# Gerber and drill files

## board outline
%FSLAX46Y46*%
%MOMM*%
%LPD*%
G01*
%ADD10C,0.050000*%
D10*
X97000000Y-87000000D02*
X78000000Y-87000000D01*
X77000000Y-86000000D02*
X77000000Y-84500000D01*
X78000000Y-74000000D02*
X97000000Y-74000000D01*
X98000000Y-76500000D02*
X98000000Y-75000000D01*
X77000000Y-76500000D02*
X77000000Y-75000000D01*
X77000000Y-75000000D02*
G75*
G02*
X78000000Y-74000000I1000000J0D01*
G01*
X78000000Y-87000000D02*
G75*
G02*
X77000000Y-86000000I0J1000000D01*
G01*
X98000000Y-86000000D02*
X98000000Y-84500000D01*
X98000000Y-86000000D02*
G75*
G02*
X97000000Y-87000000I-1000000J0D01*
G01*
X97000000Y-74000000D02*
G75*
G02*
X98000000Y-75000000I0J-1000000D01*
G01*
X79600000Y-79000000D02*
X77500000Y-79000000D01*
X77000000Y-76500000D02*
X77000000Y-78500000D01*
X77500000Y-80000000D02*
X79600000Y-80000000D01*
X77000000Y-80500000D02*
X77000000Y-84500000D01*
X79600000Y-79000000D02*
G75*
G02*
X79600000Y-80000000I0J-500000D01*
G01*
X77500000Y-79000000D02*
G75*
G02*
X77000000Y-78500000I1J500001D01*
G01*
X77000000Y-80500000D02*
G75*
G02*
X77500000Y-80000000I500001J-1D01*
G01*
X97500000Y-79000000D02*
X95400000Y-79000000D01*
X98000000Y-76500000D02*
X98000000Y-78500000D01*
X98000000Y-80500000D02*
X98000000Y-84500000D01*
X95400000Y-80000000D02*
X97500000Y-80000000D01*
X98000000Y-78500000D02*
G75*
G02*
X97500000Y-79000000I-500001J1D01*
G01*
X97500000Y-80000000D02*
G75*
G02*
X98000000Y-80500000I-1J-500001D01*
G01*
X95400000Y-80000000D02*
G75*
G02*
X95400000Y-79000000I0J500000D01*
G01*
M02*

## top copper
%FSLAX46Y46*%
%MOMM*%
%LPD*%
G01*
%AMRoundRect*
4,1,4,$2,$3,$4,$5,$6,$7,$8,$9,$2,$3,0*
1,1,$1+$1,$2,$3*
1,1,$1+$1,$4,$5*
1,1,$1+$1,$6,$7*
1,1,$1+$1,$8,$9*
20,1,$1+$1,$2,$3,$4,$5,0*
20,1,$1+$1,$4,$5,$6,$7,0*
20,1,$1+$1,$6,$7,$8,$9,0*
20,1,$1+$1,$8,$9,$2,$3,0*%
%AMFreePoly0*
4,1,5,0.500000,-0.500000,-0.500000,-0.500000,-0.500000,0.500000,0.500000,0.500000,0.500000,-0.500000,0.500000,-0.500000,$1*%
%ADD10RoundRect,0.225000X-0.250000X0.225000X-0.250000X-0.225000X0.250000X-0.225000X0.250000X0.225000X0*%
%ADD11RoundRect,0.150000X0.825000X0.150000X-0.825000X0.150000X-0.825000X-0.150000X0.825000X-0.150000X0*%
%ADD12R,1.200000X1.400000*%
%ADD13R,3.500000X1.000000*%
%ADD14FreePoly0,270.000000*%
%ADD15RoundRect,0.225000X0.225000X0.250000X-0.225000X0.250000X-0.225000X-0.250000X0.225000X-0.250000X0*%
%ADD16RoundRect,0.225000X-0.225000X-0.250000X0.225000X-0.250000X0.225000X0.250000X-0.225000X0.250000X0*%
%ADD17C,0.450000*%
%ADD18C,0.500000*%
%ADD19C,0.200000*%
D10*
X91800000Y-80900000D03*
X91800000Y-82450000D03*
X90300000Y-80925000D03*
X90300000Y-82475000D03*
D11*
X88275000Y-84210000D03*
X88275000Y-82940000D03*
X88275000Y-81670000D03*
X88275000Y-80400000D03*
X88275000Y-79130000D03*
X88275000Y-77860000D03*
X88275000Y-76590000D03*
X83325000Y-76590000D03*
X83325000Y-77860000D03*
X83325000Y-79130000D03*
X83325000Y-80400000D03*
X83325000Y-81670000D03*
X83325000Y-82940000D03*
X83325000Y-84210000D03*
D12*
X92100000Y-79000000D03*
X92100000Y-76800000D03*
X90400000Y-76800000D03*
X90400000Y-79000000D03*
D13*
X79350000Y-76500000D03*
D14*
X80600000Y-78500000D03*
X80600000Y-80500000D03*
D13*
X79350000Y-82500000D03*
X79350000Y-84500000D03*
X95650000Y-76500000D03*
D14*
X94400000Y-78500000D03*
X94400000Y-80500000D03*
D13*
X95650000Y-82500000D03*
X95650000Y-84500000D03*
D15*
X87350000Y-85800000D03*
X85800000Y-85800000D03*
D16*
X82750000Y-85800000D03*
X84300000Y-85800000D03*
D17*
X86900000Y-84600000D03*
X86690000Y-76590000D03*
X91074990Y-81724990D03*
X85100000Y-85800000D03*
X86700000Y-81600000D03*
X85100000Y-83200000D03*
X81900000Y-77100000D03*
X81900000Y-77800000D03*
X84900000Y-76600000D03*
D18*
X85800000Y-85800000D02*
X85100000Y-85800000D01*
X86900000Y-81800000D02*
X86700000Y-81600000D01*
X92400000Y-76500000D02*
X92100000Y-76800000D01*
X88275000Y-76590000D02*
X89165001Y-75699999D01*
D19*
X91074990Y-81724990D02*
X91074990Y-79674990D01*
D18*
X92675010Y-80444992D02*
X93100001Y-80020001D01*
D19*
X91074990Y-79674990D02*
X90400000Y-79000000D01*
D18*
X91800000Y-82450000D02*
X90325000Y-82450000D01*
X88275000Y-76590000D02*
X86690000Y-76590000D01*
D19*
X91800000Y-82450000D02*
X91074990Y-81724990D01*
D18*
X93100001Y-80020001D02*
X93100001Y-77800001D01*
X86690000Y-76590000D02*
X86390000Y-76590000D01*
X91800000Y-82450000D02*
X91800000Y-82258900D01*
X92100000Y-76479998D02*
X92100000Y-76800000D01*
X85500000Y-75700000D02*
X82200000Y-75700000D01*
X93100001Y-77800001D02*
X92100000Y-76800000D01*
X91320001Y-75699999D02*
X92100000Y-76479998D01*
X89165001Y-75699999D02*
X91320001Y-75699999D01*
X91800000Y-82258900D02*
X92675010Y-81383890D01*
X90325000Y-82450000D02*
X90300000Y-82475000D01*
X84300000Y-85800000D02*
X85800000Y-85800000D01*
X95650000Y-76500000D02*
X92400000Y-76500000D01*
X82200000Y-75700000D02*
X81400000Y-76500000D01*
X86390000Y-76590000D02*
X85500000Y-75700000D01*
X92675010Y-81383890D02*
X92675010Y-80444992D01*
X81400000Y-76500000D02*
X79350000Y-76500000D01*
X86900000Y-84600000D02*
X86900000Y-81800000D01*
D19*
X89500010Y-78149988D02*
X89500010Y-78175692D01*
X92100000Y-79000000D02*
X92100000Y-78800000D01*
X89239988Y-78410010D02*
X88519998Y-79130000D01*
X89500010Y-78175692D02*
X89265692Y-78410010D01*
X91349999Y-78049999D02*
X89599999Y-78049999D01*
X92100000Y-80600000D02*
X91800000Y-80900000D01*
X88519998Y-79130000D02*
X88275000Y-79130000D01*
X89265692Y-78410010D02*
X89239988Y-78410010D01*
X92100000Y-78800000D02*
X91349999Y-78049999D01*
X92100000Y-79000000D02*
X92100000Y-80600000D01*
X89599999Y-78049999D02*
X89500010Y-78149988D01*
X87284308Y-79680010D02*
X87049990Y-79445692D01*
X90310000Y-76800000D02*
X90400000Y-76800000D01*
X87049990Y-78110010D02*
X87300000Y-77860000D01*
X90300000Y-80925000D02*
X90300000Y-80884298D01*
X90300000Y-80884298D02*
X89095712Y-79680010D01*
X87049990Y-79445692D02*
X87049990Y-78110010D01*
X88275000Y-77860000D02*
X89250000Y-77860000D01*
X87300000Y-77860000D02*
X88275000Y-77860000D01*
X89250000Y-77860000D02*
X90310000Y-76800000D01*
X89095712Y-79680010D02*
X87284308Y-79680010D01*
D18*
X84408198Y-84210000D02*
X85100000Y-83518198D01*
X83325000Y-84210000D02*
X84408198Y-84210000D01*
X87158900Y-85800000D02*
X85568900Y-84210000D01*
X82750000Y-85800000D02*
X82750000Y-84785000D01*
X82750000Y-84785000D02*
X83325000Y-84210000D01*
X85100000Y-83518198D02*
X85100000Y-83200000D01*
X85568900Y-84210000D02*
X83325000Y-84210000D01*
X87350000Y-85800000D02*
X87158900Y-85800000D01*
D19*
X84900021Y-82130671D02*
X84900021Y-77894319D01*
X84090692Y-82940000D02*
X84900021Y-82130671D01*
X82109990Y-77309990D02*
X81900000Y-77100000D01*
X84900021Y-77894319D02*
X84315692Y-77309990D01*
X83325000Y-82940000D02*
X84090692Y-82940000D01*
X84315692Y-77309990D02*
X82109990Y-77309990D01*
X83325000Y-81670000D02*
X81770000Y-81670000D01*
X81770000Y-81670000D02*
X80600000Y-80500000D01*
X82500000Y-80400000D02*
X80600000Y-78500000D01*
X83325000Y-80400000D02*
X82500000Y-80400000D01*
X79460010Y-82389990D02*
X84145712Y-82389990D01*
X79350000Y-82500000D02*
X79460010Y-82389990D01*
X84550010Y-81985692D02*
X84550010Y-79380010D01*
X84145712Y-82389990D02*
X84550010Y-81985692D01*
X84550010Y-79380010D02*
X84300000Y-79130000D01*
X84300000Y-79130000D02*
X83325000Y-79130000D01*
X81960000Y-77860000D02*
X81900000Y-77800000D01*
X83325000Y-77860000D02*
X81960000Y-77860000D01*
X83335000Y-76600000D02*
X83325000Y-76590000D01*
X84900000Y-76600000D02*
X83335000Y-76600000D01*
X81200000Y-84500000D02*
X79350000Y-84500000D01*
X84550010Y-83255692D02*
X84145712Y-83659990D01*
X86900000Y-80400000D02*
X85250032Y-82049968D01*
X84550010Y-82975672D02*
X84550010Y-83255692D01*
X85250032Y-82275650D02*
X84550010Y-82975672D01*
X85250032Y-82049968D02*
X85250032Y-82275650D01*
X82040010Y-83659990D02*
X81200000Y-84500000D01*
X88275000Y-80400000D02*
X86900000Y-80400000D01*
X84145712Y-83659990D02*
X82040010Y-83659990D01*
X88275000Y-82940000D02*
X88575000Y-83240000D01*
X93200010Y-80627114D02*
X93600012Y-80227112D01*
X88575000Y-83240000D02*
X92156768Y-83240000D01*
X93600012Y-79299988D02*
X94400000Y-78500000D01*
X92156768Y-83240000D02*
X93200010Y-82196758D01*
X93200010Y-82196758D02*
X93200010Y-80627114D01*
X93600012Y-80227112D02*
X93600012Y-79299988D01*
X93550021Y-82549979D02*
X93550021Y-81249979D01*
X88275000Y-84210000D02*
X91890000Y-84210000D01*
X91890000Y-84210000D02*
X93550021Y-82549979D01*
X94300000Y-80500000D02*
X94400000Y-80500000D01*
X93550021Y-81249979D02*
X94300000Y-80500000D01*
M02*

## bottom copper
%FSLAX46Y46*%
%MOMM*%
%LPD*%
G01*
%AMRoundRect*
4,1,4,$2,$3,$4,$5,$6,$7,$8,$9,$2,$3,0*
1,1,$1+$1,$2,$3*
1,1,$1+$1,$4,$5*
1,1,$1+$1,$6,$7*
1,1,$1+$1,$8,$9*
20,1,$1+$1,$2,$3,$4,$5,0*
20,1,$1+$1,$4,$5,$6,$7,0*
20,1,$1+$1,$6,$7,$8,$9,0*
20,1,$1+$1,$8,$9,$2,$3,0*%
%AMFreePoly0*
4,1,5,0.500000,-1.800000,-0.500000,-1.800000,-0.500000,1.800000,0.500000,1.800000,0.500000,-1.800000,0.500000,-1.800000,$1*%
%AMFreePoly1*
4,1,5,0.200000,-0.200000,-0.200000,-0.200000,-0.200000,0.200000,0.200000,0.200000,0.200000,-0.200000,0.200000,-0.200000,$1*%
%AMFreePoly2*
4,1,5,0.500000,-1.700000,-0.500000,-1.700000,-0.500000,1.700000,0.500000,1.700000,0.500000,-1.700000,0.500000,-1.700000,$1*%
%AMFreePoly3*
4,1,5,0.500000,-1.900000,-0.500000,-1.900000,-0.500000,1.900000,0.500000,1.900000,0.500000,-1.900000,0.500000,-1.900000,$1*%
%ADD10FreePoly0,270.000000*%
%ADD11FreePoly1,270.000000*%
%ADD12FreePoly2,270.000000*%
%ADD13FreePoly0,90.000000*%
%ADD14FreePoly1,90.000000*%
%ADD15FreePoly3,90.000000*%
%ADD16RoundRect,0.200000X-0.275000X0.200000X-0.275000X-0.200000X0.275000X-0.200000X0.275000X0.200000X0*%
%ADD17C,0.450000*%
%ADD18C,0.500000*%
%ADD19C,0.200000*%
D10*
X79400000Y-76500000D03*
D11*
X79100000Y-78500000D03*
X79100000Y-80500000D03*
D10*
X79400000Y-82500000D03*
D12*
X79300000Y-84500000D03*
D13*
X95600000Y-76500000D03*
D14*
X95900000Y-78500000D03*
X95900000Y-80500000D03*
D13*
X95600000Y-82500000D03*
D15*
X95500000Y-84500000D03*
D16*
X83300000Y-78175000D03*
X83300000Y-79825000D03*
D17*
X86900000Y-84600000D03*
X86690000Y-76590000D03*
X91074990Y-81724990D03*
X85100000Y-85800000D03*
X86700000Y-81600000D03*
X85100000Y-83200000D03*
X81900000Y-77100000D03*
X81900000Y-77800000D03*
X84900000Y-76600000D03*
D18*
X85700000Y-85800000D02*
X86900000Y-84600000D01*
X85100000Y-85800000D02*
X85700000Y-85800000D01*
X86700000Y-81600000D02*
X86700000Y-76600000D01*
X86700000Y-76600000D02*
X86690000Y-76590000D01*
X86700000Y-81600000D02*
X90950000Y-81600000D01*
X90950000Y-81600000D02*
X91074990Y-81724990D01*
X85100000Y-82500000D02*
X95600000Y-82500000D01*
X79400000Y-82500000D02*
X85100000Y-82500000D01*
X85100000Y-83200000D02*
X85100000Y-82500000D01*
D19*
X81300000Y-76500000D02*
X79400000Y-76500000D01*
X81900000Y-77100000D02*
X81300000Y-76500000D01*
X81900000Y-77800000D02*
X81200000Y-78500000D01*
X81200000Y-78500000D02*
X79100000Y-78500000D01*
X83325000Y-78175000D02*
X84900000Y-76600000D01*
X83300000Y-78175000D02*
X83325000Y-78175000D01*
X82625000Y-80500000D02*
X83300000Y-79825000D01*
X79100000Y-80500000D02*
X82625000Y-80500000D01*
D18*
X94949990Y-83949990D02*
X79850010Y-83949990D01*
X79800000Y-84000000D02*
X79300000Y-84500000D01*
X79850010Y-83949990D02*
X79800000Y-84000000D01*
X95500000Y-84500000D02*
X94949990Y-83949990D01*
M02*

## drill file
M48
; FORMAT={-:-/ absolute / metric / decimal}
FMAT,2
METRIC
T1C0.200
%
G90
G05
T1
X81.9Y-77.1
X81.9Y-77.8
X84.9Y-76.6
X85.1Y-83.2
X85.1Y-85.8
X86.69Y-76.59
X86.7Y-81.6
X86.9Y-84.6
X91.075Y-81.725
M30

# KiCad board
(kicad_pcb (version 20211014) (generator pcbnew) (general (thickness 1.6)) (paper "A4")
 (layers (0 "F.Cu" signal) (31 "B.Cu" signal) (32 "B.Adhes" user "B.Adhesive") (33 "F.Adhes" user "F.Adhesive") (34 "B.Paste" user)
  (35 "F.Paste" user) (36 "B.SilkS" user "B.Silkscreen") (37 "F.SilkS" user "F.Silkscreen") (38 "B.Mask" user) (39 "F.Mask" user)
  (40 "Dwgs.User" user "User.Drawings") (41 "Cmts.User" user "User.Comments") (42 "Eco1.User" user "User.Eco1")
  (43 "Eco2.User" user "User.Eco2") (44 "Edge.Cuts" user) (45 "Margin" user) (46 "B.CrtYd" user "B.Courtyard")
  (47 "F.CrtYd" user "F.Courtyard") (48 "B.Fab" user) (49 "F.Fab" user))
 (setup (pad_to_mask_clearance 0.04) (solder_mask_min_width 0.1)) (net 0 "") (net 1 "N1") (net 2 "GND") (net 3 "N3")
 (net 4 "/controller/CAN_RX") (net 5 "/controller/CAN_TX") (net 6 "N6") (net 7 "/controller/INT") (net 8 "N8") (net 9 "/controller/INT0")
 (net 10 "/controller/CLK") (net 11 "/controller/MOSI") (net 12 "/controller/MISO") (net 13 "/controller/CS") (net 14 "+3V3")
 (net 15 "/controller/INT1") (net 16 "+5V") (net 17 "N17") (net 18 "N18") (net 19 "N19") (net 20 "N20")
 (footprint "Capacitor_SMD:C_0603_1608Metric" (layer "F.Cu") (at 91.8 81.675 -90)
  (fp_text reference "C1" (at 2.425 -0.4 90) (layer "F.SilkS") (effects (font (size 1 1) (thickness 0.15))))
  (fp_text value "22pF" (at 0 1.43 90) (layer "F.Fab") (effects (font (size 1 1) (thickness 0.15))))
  (pad "1" smd roundrect locked (at -0.775 0 270) (size 0.9 0.95) (layers "F.Cu" "F.Paste" "F.Mask") (roundrect_rratio 0.25) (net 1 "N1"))
  (pad "2" smd roundrect locked (at 0.775 0 270) (size 0.9 0.95) (layers "F.Cu" "F.Paste" "F.Mask") (roundrect_rratio 0.25) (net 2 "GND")))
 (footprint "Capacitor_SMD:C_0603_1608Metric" (layer "F.Cu") (at 90.3 81.7 -90)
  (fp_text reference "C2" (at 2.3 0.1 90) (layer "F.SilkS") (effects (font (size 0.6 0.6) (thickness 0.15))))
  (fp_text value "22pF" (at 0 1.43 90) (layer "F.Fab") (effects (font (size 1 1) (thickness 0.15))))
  (pad "1" smd roundrect locked (at -0.775 0 270) (size 0.9 0.95) (layers "F.Cu" "F.Paste" "F.Mask") (roundrect_rratio 0.25) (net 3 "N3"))
  (pad "2" smd roundrect locked (at 0.775 0 270) (size 0.9 0.95) (layers "F.Cu" "F.Paste" "F.Mask") (roundrect_rratio 0.25) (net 2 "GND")))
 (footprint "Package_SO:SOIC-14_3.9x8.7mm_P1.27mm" (layer "F.Cu") (at 85.8 80.4 180)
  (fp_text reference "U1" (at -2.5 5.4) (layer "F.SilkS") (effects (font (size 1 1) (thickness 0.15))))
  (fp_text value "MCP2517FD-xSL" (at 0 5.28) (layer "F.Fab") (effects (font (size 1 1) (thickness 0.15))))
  (pad "1" smd roundrect locked (at -2.475 -3.81 180) (size 1.95 0.6) (layers "F.Cu" "F.Paste" "F.Mask") (roundrect_rratio 0.25)
   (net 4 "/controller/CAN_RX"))
  (pad "2" smd roundrect locked (at -2.475 -2.54 180) (size 1.95 0.6) (layers "F.Cu" "F.Paste" "F.Mask") (roundrect_rratio 0.25)
   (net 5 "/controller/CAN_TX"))
  (pad "3" smd roundrect locked (at -2.475 -1.27 180) (size 1.95 0.6) (layers "F.Cu" "F.Paste" "F.Mask") (roundrect_rratio 0.25)
   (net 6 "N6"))
  (pad "4" smd roundrect locked (at -2.475 0 180) (size 1.95 0.6) (layers "F.Cu" "F.Paste" "F.Mask") (roundrect_rratio 0.25)
   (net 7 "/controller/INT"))
  (pad "5" smd roundrect locked (at -2.475 1.27 180) (size 1.95 0.6) (layers "F.Cu" "F.Paste" "F.Mask") (roundrect_rratio 0.25) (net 1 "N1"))
  (pad "6" smd roundrect locked (at -2.475 2.54 180) (size 1.95 0.6) (layers "F.Cu" "F.Paste" "F.Mask") (roundrect_rratio 0.25) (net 3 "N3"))
  (pad "7" smd roundrect locked (at -2.475 3.81 180) (size 1.95 0.6) (layers "F.Cu" "F.Paste" "F.Mask") (roundrect_rratio 0.25)
   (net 2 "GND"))
  (pad "8" smd roundrect locked (at 2.475 3.81 180) (size 1.95 0.6) (layers "F.Cu" "F.Paste" "F.Mask") (roundrect_rratio 0.25) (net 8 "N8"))
  (pad "9" smd roundrect locked (at 2.475 2.54 180) (size 1.95 0.6) (layers "F.Cu" "F.Paste" "F.Mask") (roundrect_rratio 0.25)
   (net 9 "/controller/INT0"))
  (pad "10" smd roundrect locked (at 2.475 1.27 180) (size 1.95 0.6) (layers "F.Cu" "F.Paste" "F.Mask") (roundrect_rratio 0.25)
   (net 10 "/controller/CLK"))
  (pad "11" smd roundrect locked (at 2.475 0 180) (size 1.95 0.6) (layers "F.Cu" "F.Paste" "F.Mask") (roundrect_rratio 0.25)
   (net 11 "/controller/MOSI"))
  (pad "12" smd roundrect locked (at 2.475 -1.27 180) (size 1.95 0.6) (layers "F.Cu" "F.Paste" "F.Mask") (roundrect_rratio 0.25)
   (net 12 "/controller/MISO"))
  (pad "13" smd roundrect locked (at 2.475 -2.54 180) (size 1.95 0.6) (layers "F.Cu" "F.Paste" "F.Mask") (roundrect_rratio 0.25)
   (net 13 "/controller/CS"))
  (pad "14" smd roundrect locked (at 2.475 -3.81 180) (size 1.95 0.6) (layers "F.Cu" "F.Paste" "F.Mask") (roundrect_rratio 0.25)
   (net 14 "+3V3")))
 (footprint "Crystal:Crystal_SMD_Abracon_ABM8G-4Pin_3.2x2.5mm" (layer "F.Cu") (at 91.25 77.9 90)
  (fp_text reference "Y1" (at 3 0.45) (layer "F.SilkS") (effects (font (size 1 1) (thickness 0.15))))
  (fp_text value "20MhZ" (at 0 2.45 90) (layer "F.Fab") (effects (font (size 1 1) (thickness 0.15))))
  (pad "1" smd rect locked (at -1.1 0.85 90) (size 1.4 1.2) (layers "F.Cu" "F.Paste" "F.Mask") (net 1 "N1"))
  (pad "2" smd rect locked (at 1.1 0.85 90) (size 1.4 1.2) (layers "F.Cu" "F.Paste" "F.Mask") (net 2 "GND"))
  (pad "3" smd rect locked (at 1.1 -0.85 90) (size 1.4 1.2) (layers "F.Cu" "F.Paste" "F.Mask") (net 3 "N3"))
  (pad "4" smd rect locked (at -1.1 -0.85 90) (size 1.4 1.2) (layers "F.Cu" "F.Paste" "F.Mask") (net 2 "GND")))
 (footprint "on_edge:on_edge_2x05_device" (layer "F.Cu") (at 77 80.5 -90)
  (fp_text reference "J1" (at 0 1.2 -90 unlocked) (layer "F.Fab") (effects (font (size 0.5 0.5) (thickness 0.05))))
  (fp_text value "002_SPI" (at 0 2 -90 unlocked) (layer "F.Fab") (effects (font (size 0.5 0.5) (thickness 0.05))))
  (fp_line (start -1.5 -2.6) (end -1.5 -0.5) (layer "Edge.Cuts") (width 0.05))
  (fp_line (start -4 0) (end -2 0) (layer "Edge.Cuts") (width 0.05))
  (fp_line (start -0.5 -0.5) (end -0.5 -2.6) (layer "Edge.Cuts") (width 0.05))
  (fp_line (start 0 0) (end 4 0) (layer "Edge.Cuts") (width 0.05))
  (fp_arc (start -1.5 -2.6) (mid -1 -3.1) (end -0.5 -2.6) (layer "Edge.Cuts") (width 0.05))
  (fp_arc (start -1.5 -0.5) (mid -1.646447 -0.146447) (end -2 0) (layer "Edge.Cuts") (width 0.05))
  (fp_arc (start 0 0) (mid -0.353553 -0.146447) (end -0.5 -0.5) (layer "Edge.Cuts") (width 0.05))
  (pad "1" smd rect locked (at -4 -2.35 90) (size 1 3.5) (layers "F.Cu" "F.Mask") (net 2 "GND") (zone_connect 0))
  (pad "2" smd custom locked (at -2 -3.6 270) (size 1 1) (layers "F.Cu" "F.Mask") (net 11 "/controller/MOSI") (zone_connect 0)
   (options (clearance outline) (anchor rect)) (primitives))
  (pad "3" smd custom locked (at 0 -3.6 270) (size 1 1) (layers "F.Cu" "F.Mask") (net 12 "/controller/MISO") (zone_connect 0)
   (options (clearance outline) (anchor rect)) (primitives))
  (pad "4" smd rect locked (at 2 -2.35 90) (size 1 3.5) (layers "F.Cu" "F.Mask") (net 10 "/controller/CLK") (zone_connect 0))
  (pad "5" smd rect locked (at 4 -2.35 90) (size 1 3.5) (layers "F.Cu" "F.Mask") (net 7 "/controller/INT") (zone_connect 0))
  (pad "6" smd custom locked (at -4 -2.4 270) (size 1 3.6) (layers "B.Cu" "B.Mask") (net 13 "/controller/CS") (zone_connect 0)
   (options (clearance outline) (anchor rect)) (primitives))
  (pad "7" smd custom locked (at -2 -2.1 270) (size 0.4 0.4) (layers "B.Cu" "B.Mask") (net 9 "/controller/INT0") (zone_connect 0)
   (options (clearance outline) (anchor rect)) (primitives))
  (pad "8" smd custom locked (at 0 -2.1 270) (size 0.4 0.4) (layers "B.Cu" "B.Mask") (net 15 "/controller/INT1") (zone_connect 0)
   (options (clearance outline) (anchor rect)) (primitives))
  (pad "9" smd custom locked (at 2 -2.4 270) (size 1 3.6) (layers "B.Cu" "B.Mask") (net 14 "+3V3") (zone_connect 0)
   (options (clearance outline) (anchor rect)) (primitives))
  (pad "10" smd custom locked (at 4 -2.3 270) (size 1 3.4) (layers "B.Cu" "B.Mask") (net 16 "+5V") (zone_connect 0)
   (options (clearance outline) (anchor rect)) (primitives)))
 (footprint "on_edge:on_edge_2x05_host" (layer "F.Cu") (at 98 80.5 -90)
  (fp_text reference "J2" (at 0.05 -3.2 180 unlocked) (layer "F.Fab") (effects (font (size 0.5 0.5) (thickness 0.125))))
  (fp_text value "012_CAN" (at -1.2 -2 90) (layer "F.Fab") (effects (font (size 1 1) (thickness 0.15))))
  (fp_line (start -1.5 0.5) (end -1.5 2.6) (layer "Edge.Cuts") (width 0.05))
  (fp_line (start -4 0) (end -2 0) (layer "Edge.Cuts") (width 0.05))
  (fp_line (start 0 0) (end 4 0) (layer "Edge.Cuts") (width 0.05))
  (fp_line (start -0.5 2.6) (end -0.5 0.5) (layer "Edge.Cuts") (width 0.05))
  (fp_arc (start -2 0) (mid -1.646447 0.146447) (end -1.5 0.5) (layer "Edge.Cuts") (width 0.05))
  (fp_arc (start -0.5 0.5) (mid -0.353553 0.146447) (end 0 0) (layer "Edge.Cuts") (width 0.05))
  (fp_arc (start -0.5 2.6) (mid -1 3.1) (end -1.5 2.6) (layer "Edge.Cuts") (width 0.05))
  (pad "1" smd rect locked (at -4 2.35 270) (size 1 3.5) (layers "F.Cu" "F.Mask") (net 2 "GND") (zone_connect 0))
  (pad "2" smd custom locked (at -2 3.6 270) (size 1 1) (layers "F.Cu" "F.Mask") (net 5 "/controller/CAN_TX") (zone_connect 0)
   (options (clearance outline) (anchor rect)) (primitives))
  (pad "3" smd custom locked (at 0 3.6 270) (size 1 1) (layers "F.Cu" "F.Mask") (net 4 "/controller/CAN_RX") (zone_connect 0)
   (options (clearance outline) (anchor rect)) (primitives))
  (pad "4" smd rect locked (at 2 2.35 270) (size 1 3.5) (layers "F.Cu" "F.Mask") (zone_connect 0))
  (pad "5" smd rect locked (at 4 2.35 270) (size 1 3.5) (layers "F.Cu" "F.Mask") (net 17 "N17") (zone_connect 0))
  (pad "6" smd custom locked (at -4 2.4 90) (size 1 3.6) (layers "B.Cu" "B.Mask") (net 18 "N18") (zone_connect 0)
   (options (clearance outline) (anchor rect)) (primitives))
  (pad "7" smd custom locked (at -2 2.1 90) (size 0.4 0.4) (layers "B.Cu" "B.Mask") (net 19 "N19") (zone_connect 0)
   (options (clearance outline) (anchor rect)) (primitives))
  (pad "8" smd custom locked (at 0 2.1 90) (size 0.4 0.4) (layers "B.Cu" "B.Mask") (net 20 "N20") (zone_connect 0)
   (options (clearance outline) (anchor rect)) (primitives))
  (pad "9" smd custom locked (at 2 2.4 90) (size 1 3.6) (layers "B.Cu" "B.Mask") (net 14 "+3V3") (zone_connect 0)
   (options (clearance outline) (anchor rect)) (primitives))
  (pad "10" smd custom locked (at 4 2.5 90) (size 1 3.8) (layers "B.Cu" "B.Mask") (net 16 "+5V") (zone_connect 0)
   (options (clearance outline) (anchor rect)) (primitives)))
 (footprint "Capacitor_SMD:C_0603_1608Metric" (layer "F.Cu") (at 86.575 85.8 180)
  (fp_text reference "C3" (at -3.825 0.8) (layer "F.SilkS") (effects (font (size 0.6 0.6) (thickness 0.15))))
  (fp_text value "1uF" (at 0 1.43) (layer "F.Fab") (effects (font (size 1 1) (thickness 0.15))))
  (pad "1" smd roundrect locked (at -0.775 0 180) (size 0.9 0.95) (layers "F.Cu" "F.Paste" "F.Mask") (roundrect_rratio 0.25) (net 14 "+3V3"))
  (pad "2" smd roundrect locked (at 0.775 0 180) (size 0.9 0.95) (layers "F.Cu" "F.Paste" "F.Mask") (roundrect_rratio 0.25) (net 2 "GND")))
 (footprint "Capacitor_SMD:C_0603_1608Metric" (layer "F.Cu") (at 83.525 85.8)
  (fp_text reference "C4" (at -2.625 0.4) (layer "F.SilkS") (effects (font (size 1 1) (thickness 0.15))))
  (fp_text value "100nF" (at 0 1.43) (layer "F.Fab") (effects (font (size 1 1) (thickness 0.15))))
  (pad "1" smd roundrect locked (at -0.775 0) (size 0.9 0.95) (layers "F.Cu" "F.Paste" "F.Mask") (roundrect_rratio 0.25) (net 14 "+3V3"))
  (pad "2" smd roundrect locked (at 0.775 0) (size 0.9 0.95) (layers "F.Cu" "F.Paste" "F.Mask") (roundrect_rratio 0.25) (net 2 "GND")))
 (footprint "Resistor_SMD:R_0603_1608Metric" (layer "B.Cu") (at 83.3 79 -90)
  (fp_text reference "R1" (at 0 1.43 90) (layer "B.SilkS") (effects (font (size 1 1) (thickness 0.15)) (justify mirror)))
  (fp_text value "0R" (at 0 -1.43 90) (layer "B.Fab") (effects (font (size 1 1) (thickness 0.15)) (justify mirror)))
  (pad "1" smd roundrect locked (at -0.825 0 270) (size 0.8 0.95) (layers "B.Cu" "B.Paste" "B.Mask") (roundrect_rratio 0.25) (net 8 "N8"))
  (pad "2" smd roundrect locked (at 0.825 0 270) (size 0.8 0.95) (layers "B.Cu" "B.Paste" "B.Mask") (roundrect_rratio 0.25)
   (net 15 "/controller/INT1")))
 (gr_line (start 97 87) (end 78 87) (layer "Edge.Cuts") (width 0.05))
 (gr_line (start 77 86) (end 77 84.5) (layer "Edge.Cuts") (width 0.05))
 (gr_line (start 78 74) (end 97 74) (layer "Edge.Cuts") (width 0.05))
 (gr_line (start 98 76.5) (end 98 75) (layer "Edge.Cuts") (width 0.05))
 (gr_line (start 77 76.5) (end 77 75) (layer "Edge.Cuts") (width 0.05))
 (gr_arc (start 77 75) (mid 77.292893 74.292893) (end 78 74) (layer "Edge.Cuts") (width 0.05))
 (gr_arc (start 78 87) (mid 77.292893 86.707107) (end 77 86) (layer "Edge.Cuts") (width 0.05))
 (gr_line (start 98 86) (end 98 84.5) (layer "Edge.Cuts") (width 0.05))
 (gr_arc (start 98 86) (mid 97.707107 86.707107) (end 97 87) (layer "Edge.Cuts") (width 0.05))
 (gr_arc (start 97 74) (mid 97.707107 74.292893) (end 98 75) (layer "Edge.Cuts") (width 0.05))
 (segment (start 85.8 85.8) (end 85.1 85.8) (width 0.5) (layer "F.Cu") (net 2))
 (segment (start 86.9 81.8) (end 86.7 81.6) (width 0.5) (layer "F.Cu") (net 2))
 (segment (start 92.4 76.5) (end 92.1 76.8) (width 0.5) (layer "F.Cu") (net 2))
 (segment (start 88.275 76.59) (end 89.165001 75.699999) (width 0.5) (layer "F.Cu") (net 2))
 (segment (start 91.07499 81.72499) (end 91.07499 79.67499) (width 0.2) (layer "F.Cu") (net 2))
 (segment (start 92.67501 80.444992) (end 93.100001 80.020001) (width 0.5) (layer "F.Cu") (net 2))
 (segment (start 91.07499 79.67499) (end 90.4 79) (width 0.2) (layer "F.Cu") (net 2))
 (segment (start 91.8 82.45) (end 90.325 82.45) (width 0.5) (layer "F.Cu") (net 2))
 (segment (start 88.275 76.59) (end 86.69 76.59) (width 0.5) (layer "F.Cu") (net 2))
 (segment (start 91.8 82.45) (end 91.07499 81.72499) (width 0.2) (layer "F.Cu") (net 2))
 (segment (start 93.100001 80.020001) (end 93.100001 77.800001) (width 0.5) (layer "F.Cu") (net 2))
 (segment (start 86.69 76.59) (end 86.39 76.59) (width 0.5) (layer "F.Cu") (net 2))
 (segment (start 91.8 82.45) (end 91.8 82.2589) (width 0.5) (layer "F.Cu") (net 2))
 (segment (start 92.1 76.479998) (end 92.1 76.8) (width 0.5) (layer "F.Cu") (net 2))
 (segment (start 85.5 75.7) (end 82.2 75.7) (width 0.5) (layer "F.Cu") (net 2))
 (segment (start 93.100001 77.800001) (end 92.1 76.8) (width 0.5) (layer "F.Cu") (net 2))
 (segment (start 91.320001 75.699999) (end 92.1 76.479998) (width 0.5) (layer "F.Cu") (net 2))
 (segment (start 89.165001 75.699999) (end 91.320001 75.699999) (width 0.5) (layer "F.Cu") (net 2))
 (segment (start 91.8 82.2589) (end 92.67501 81.38389) (width 0.5) (layer "F.Cu") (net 2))
 (segment (start 90.325 82.45) (end 90.3 82.475) (width 0.5) (layer "F.Cu") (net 2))
 (segment (start 84.3 85.8) (end 85.8 85.8) (width 0.5) (layer "F.Cu") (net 2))
 (segment (start 95.65 76.5) (end 92.4 76.5) (width 0.5) (layer "F.Cu") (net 2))
 (segment (start 82.2 75.7) (end 81.4 76.5) (width 0.5) (layer "F.Cu") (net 2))
 (segment (start 86.39 76.59) (end 85.5 75.7) (width 0.5) (layer "F.Cu") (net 2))
 (segment (start 92.67501 81.38389) (end 92.67501 80.444992) (width 0.5) (layer "F.Cu") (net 2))
 (segment (start 81.4 76.5) (end 79.35 76.5) (width 0.5) (layer "F.Cu") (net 2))
 (segment (start 86.9 84.6) (end 86.9 81.8) (width 0.5) (layer "F.Cu") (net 2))
 (via (at 86.9 84.6) (size 0.45) (drill 0.2) (layers "F.Cu" "B.Cu") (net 2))
 (via (at 86.69 76.59) (size 0.45) (drill 0.2) (layers "F.Cu" "B.Cu") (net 2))
 (via (at 91.07499 81.72499) (size 0.45) (drill 0.2) (layers "F.Cu" "B.Cu") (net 2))
 (via (at 85.1 85.8) (size 0.45) (drill 0.2) (layers "F.Cu" "B.Cu") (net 2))
 (via (at 86.7 81.6) (size 0.45) (drill 0.2) (layers "F.Cu" "B.Cu") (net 2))
 (segment (start 85.7 85.8) (end 86.9 84.6) (width 0.5) (layer "B.Cu") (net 2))
 (segment (start 85.1 85.8) (end 85.7 85.8) (width 0.5) (layer "B.Cu") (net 2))
 (segment (start 86.7 81.6) (end 86.7 76.6) (width 0.5) (layer "B.Cu") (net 2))
 (segment (start 86.7 76.6) (end 86.69 76.59) (width 0.5) (layer "B.Cu") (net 2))
 (segment (start 86.7 81.6) (end 90.95 81.6) (width 0.5) (layer "B.Cu") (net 2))
 (segment (start 90.95 81.6) (end 91.07499 81.72499) (width 0.5) (layer "B.Cu") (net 2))
 (segment (start 89.50001 78.149988) (end 89.50001 78.175692) (width 0.2) (layer "F.Cu") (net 1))
 (segment (start 92.1 79) (end 92.1 78.8) (width 0.2) (layer "F.Cu") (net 1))
 (segment (start 89.239988 78.41001) (end 88.519998 79.13) (width 0.2) (layer "F.Cu") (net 1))
 (segment (start 89.50001 78.175692) (end 89.265692 78.41001) (width 0.2) (layer "F.Cu") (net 1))
 (segment (start 91.349999 78.049999) (end 89.599999 78.049999) (width 0.2) (layer "F.Cu") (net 1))
 (segment (start 92.1 80.6) (end 91.8 80.9) (width 0.2) (layer "F.Cu") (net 1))
 (segment (start 88.519998 79.13) (end 88.275 79.13) (width 0.2) (layer "F.Cu") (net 1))
 (segment (start 89.265692 78.41001) (end 89.239988 78.41001) (width 0.2) (layer "F.Cu") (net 1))
 (segment (start 92.1 78.8) (end 91.349999 78.049999) (width 0.2) (layer "F.Cu") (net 1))
 (segment (start 92.1 79) (end 92.1 80.6) (width 0.2) (layer "F.Cu") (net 1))
 (segment (start 89.599999 78.049999) (end 89.50001 78.149988) (width 0.2) (layer "F.Cu") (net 1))
 (segment (start 87.284308 79.68001) (end 87.04999 79.445692) (width 0.2) (layer "F.Cu") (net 3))
 (segment (start 90.31 76.8) (end 90.4 76.8) (width 0.2) (layer "F.Cu") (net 3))
 (segment (start 87.04999 78.11001) (end 87.3 77.86) (width 0.2) (layer "F.Cu") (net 3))
 (segment (start 90.3 80.925) (end 90.3 80.884298) (width 0.2) (layer "F.Cu") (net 3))
 (segment (start 90.3 80.884298) (end 89.095712 79.68001) (width 0.2) (layer "F.Cu") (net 3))
 (segment (start 87.04999 79.445692) (end 87.04999 78.11001) (width 0.2) (layer "F.Cu") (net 3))
 (segment (start 88.275 77.86) (end 89.25 77.86) (width 0.2) (layer "F.Cu") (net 3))
 (segment (start 87.3 77.86) (end 88.275 77.86) (width 0.2) (layer "F.Cu") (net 3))
 (segment (start 89.25 77.86) (end 90.31 76.8) (width 0.2) (layer "F.Cu") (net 3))
 (segment (start 89.095712 79.68001) (end 87.284308 79.68001) (width 0.2) (layer "F.Cu") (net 3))
 (segment (start 84.408198 84.21) (end 85.1 83.518198) (width 0.5) (layer "F.Cu") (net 14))
 (segment (start 83.325 84.21) (end 84.408198 84.21) (width 0.5) (layer "F.Cu") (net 14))
 (segment (start 87.1589 85.8) (end 85.5689 84.21) (width 0.5) (layer "F.Cu") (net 14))
 (segment (start 82.75 85.8) (end 82.75 84.785) (width 0.5) (layer "F.Cu") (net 14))
 (segment (start 82.75 84.785) (end 83.325 84.21) (width 0.5) (layer "F.Cu") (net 14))
 (segment (start 85.1 83.518198) (end 85.1 83.2) (width 0.5) (layer "F.Cu") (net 14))
 (segment (start 85.5689 84.21) (end 83.325 84.21) (width 0.5) (layer "F.Cu") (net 14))
 (segment (start 87.35 85.8) (end 87.1589 85.8) (width 0.5) (layer "F.Cu") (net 14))
 (via (at 85.1 83.2) (size 0.45) (drill 0.2) (layers "F.Cu" "B.Cu") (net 14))
 (segment (start 85.1 82.5) (end 95.6 82.5) (width 0.5) (layer "B.Cu") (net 14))
 (segment (start 79.4 82.5) (end 85.1 82.5) (width 0.5) (layer "B.Cu") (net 14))
 (segment (start 85.1 83.2) (end 85.1 82.5) (width 0.5) (layer "B.Cu") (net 14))
 (segment (start 84.900021 82.130671) (end 84.900021 77.894319) (width 0.2) (layer "F.Cu") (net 13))
 (segment (start 84.090692 82.94) (end 84.900021 82.130671) (width 0.2) (layer "F.Cu") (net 13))
 (segment (start 82.10999 77.30999) (end 81.9 77.1) (width 0.2) (layer "F.Cu") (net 13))
 (segment (start 84.900021 77.894319) (end 84.315692 77.30999) (width 0.2) (layer "F.Cu") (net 13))
 (segment (start 83.325 82.94) (end 84.090692 82.94) (width 0.2) (layer "F.Cu") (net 13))
 (segment (start 84.315692 77.30999) (end 82.10999 77.30999) (width 0.2) (layer "F.Cu") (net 13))
 (via (at 81.9 77.1) (size 0.45) (drill 0.2) (layers "F.Cu" "B.Cu") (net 13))
 (segment (start 81.3 76.5) (end 79.4 76.5) (width 0.2) (layer "B.Cu") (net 13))
 (segment (start 81.9 77.1) (end 81.3 76.5) (width 0.2) (layer "B.Cu") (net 13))
 (segment (start 83.325 81.67) (end 81.77 81.67) (width 0.2) (layer "F.Cu") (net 12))
 (segment (start 81.77 81.67) (end 80.6 80.5) (width 0.2) (layer "F.Cu") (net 12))
 (segment (start 82.5 80.4) (end 80.6 78.5) (width 0.2) (layer "F.Cu") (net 11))
 (segment (start 83.325 80.4) (end 82.5 80.4) (width 0.2) (layer "F.Cu") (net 11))
 (segment (start 79.46001 82.38999) (end 84.145712 82.38999) (width 0.2) (layer "F.Cu") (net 10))
 (segment (start 79.35 82.5) (end 79.46001 82.38999) (width 0.2) (layer "F.Cu") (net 10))
 (segment (start 84.55001 81.985692) (end 84.55001 79.38001) (width 0.2) (layer "F.Cu") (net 10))
 (segment (start 84.145712 82.38999) (end 84.55001 81.985692) (width 0.2) (layer "F.Cu") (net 10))
 (segment (start 84.55001 79.38001) (end 84.3 79.13) (width 0.2) (layer "F.Cu") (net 10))
 (segment (start 84.3 79.13) (end 83.325 79.13) (width 0.2) (layer "F.Cu") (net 10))
 (segment (start 81.96 77.86) (end 81.9 77.8) (width 0.2) (layer "F.Cu") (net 9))
 (segment (start 83.325 77.86) (end 81.96 77.86) (width 0.2) (layer "F.Cu") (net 9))
 (via (at 81.9 77.8) (size 0.45) (drill 0.2) (layers "F.Cu" "B.Cu") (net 9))
 (segment (start 81.9 77.8) (end 81.2 78.5) (width 0.2) (layer "B.Cu") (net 9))
 (segment (start 81.2 78.5) (end 79.1 78.5) (width 0.2) (layer "B.Cu") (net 9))
 (segment (start 83.335 76.6) (end 83.325 76.59) (width 0.2) (layer "F.Cu") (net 8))
 (segment (start 84.9 76.6) (end 83.335 76.6) (width 0.2) (layer "F.Cu") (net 8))
 (via (at 84.9 76.6) (size 0.45) (drill 0.2) (layers "F.Cu" "B.Cu") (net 8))
 (segment (start 83.325 78.175) (end 84.9 76.6) (width 0.2) (layer "B.Cu") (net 8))
 (segment (start 83.3 78.175) (end 83.325 78.175) (width 0.2) (layer "B.Cu") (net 8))
 (segment (start 81.2 84.5) (end 79.35 84.5) (width 0.2) (layer "F.Cu") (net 7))
 (segment (start 84.55001 83.255692) (end 84.145712 83.65999) (width 0.2) (layer "F.Cu") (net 7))
 (segment (start 86.9 80.4) (end 85.250032 82.049968) (width 0.2) (layer "F.Cu") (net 7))
 (segment (start 84.55001 82.975672) (end 84.55001 83.255692) (width 0.2) (layer "F.Cu") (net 7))
 (segment (start 85.250032 82.27565) (end 84.55001 82.975672) (width 0.2) (layer "F.Cu") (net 7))
 (segment (start 85.250032 82.049968) (end 85.250032 82.27565) (width 0.2) (layer "F.Cu") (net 7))
 (segment (start 82.04001 83.65999) (end 81.2 84.5) (width 0.2) (layer "F.Cu") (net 7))
 (segment (start 88.275 80.4) (end 86.9 80.4) (width 0.2) (layer "F.Cu") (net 7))
 (segment (start 84.145712 83.65999) (end 82.04001 83.65999) (width 0.2) (layer "F.Cu") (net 7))
 (segment (start 88.275 82.94) (end 88.575 83.24) (width 0.2) (layer "F.Cu") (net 5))
 (segment (start 93.20001 80.627114) (end 93.600012 80.227112) (width 0.2) (layer "F.Cu") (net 5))
 (segment (start 88.575 83.24) (end 92.156768 83.24) (width 0.2) (layer "F.Cu") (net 5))
 (segment (start 93.600012 79.299988) (end 94.4 78.5) (width 0.2) (layer "F.Cu") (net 5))
 (segment (start 92.156768 83.24) (end 93.20001 82.196758) (width 0.2) (layer "F.Cu") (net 5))
 (segment (start 93.20001 82.196758) (end 93.20001 80.627114) (width 0.2) (layer "F.Cu") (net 5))
 (segment (start 93.600012 80.227112) (end 93.600012 79.299988) (width 0.2) (layer "F.Cu") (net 5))
 (segment (start 93.550021 82.549979) (end 93.550021 81.249979) (width 0.2) (layer "F.Cu") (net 4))
 (segment (start 88.275 84.21) (end 91.89 84.21) (width 0.2) (layer "F.Cu") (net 4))
 (segment (start 91.89 84.21) (end 93.550021 82.549979) (width 0.2) (layer "F.Cu") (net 4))
 (segment (start 94.3 80.5) (end 94.4 80.5) (width 0.2) (layer "F.Cu") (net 4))
 (segment (start 93.550021 81.249979) (end 94.3 80.5) (width 0.2) (layer "F.Cu") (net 4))
 (segment (start 82.625 80.5) (end 83.3 79.825) (width 0.2) (layer "B.Cu") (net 15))
 (segment (start 79.1 80.5) (end 82.625 80.5) (width 0.2) (layer "B.Cu") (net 15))
 (segment (start 94.94999 83.94999) (end 79.85001 83.94999) (width 0.5) (layer "B.Cu") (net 16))
 (segment (start 79.8 84) (end 79.3 84.5) (width 0.5) (layer "B.Cu") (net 16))
 (segment (start 79.85001 83.94999) (end 79.8 84) (width 0.5) (layer "B.Cu") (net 16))
 (segment (start 95.5 84.5) (end 94.94999 83.94999) (width 0.5) (layer "B.Cu") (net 16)))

